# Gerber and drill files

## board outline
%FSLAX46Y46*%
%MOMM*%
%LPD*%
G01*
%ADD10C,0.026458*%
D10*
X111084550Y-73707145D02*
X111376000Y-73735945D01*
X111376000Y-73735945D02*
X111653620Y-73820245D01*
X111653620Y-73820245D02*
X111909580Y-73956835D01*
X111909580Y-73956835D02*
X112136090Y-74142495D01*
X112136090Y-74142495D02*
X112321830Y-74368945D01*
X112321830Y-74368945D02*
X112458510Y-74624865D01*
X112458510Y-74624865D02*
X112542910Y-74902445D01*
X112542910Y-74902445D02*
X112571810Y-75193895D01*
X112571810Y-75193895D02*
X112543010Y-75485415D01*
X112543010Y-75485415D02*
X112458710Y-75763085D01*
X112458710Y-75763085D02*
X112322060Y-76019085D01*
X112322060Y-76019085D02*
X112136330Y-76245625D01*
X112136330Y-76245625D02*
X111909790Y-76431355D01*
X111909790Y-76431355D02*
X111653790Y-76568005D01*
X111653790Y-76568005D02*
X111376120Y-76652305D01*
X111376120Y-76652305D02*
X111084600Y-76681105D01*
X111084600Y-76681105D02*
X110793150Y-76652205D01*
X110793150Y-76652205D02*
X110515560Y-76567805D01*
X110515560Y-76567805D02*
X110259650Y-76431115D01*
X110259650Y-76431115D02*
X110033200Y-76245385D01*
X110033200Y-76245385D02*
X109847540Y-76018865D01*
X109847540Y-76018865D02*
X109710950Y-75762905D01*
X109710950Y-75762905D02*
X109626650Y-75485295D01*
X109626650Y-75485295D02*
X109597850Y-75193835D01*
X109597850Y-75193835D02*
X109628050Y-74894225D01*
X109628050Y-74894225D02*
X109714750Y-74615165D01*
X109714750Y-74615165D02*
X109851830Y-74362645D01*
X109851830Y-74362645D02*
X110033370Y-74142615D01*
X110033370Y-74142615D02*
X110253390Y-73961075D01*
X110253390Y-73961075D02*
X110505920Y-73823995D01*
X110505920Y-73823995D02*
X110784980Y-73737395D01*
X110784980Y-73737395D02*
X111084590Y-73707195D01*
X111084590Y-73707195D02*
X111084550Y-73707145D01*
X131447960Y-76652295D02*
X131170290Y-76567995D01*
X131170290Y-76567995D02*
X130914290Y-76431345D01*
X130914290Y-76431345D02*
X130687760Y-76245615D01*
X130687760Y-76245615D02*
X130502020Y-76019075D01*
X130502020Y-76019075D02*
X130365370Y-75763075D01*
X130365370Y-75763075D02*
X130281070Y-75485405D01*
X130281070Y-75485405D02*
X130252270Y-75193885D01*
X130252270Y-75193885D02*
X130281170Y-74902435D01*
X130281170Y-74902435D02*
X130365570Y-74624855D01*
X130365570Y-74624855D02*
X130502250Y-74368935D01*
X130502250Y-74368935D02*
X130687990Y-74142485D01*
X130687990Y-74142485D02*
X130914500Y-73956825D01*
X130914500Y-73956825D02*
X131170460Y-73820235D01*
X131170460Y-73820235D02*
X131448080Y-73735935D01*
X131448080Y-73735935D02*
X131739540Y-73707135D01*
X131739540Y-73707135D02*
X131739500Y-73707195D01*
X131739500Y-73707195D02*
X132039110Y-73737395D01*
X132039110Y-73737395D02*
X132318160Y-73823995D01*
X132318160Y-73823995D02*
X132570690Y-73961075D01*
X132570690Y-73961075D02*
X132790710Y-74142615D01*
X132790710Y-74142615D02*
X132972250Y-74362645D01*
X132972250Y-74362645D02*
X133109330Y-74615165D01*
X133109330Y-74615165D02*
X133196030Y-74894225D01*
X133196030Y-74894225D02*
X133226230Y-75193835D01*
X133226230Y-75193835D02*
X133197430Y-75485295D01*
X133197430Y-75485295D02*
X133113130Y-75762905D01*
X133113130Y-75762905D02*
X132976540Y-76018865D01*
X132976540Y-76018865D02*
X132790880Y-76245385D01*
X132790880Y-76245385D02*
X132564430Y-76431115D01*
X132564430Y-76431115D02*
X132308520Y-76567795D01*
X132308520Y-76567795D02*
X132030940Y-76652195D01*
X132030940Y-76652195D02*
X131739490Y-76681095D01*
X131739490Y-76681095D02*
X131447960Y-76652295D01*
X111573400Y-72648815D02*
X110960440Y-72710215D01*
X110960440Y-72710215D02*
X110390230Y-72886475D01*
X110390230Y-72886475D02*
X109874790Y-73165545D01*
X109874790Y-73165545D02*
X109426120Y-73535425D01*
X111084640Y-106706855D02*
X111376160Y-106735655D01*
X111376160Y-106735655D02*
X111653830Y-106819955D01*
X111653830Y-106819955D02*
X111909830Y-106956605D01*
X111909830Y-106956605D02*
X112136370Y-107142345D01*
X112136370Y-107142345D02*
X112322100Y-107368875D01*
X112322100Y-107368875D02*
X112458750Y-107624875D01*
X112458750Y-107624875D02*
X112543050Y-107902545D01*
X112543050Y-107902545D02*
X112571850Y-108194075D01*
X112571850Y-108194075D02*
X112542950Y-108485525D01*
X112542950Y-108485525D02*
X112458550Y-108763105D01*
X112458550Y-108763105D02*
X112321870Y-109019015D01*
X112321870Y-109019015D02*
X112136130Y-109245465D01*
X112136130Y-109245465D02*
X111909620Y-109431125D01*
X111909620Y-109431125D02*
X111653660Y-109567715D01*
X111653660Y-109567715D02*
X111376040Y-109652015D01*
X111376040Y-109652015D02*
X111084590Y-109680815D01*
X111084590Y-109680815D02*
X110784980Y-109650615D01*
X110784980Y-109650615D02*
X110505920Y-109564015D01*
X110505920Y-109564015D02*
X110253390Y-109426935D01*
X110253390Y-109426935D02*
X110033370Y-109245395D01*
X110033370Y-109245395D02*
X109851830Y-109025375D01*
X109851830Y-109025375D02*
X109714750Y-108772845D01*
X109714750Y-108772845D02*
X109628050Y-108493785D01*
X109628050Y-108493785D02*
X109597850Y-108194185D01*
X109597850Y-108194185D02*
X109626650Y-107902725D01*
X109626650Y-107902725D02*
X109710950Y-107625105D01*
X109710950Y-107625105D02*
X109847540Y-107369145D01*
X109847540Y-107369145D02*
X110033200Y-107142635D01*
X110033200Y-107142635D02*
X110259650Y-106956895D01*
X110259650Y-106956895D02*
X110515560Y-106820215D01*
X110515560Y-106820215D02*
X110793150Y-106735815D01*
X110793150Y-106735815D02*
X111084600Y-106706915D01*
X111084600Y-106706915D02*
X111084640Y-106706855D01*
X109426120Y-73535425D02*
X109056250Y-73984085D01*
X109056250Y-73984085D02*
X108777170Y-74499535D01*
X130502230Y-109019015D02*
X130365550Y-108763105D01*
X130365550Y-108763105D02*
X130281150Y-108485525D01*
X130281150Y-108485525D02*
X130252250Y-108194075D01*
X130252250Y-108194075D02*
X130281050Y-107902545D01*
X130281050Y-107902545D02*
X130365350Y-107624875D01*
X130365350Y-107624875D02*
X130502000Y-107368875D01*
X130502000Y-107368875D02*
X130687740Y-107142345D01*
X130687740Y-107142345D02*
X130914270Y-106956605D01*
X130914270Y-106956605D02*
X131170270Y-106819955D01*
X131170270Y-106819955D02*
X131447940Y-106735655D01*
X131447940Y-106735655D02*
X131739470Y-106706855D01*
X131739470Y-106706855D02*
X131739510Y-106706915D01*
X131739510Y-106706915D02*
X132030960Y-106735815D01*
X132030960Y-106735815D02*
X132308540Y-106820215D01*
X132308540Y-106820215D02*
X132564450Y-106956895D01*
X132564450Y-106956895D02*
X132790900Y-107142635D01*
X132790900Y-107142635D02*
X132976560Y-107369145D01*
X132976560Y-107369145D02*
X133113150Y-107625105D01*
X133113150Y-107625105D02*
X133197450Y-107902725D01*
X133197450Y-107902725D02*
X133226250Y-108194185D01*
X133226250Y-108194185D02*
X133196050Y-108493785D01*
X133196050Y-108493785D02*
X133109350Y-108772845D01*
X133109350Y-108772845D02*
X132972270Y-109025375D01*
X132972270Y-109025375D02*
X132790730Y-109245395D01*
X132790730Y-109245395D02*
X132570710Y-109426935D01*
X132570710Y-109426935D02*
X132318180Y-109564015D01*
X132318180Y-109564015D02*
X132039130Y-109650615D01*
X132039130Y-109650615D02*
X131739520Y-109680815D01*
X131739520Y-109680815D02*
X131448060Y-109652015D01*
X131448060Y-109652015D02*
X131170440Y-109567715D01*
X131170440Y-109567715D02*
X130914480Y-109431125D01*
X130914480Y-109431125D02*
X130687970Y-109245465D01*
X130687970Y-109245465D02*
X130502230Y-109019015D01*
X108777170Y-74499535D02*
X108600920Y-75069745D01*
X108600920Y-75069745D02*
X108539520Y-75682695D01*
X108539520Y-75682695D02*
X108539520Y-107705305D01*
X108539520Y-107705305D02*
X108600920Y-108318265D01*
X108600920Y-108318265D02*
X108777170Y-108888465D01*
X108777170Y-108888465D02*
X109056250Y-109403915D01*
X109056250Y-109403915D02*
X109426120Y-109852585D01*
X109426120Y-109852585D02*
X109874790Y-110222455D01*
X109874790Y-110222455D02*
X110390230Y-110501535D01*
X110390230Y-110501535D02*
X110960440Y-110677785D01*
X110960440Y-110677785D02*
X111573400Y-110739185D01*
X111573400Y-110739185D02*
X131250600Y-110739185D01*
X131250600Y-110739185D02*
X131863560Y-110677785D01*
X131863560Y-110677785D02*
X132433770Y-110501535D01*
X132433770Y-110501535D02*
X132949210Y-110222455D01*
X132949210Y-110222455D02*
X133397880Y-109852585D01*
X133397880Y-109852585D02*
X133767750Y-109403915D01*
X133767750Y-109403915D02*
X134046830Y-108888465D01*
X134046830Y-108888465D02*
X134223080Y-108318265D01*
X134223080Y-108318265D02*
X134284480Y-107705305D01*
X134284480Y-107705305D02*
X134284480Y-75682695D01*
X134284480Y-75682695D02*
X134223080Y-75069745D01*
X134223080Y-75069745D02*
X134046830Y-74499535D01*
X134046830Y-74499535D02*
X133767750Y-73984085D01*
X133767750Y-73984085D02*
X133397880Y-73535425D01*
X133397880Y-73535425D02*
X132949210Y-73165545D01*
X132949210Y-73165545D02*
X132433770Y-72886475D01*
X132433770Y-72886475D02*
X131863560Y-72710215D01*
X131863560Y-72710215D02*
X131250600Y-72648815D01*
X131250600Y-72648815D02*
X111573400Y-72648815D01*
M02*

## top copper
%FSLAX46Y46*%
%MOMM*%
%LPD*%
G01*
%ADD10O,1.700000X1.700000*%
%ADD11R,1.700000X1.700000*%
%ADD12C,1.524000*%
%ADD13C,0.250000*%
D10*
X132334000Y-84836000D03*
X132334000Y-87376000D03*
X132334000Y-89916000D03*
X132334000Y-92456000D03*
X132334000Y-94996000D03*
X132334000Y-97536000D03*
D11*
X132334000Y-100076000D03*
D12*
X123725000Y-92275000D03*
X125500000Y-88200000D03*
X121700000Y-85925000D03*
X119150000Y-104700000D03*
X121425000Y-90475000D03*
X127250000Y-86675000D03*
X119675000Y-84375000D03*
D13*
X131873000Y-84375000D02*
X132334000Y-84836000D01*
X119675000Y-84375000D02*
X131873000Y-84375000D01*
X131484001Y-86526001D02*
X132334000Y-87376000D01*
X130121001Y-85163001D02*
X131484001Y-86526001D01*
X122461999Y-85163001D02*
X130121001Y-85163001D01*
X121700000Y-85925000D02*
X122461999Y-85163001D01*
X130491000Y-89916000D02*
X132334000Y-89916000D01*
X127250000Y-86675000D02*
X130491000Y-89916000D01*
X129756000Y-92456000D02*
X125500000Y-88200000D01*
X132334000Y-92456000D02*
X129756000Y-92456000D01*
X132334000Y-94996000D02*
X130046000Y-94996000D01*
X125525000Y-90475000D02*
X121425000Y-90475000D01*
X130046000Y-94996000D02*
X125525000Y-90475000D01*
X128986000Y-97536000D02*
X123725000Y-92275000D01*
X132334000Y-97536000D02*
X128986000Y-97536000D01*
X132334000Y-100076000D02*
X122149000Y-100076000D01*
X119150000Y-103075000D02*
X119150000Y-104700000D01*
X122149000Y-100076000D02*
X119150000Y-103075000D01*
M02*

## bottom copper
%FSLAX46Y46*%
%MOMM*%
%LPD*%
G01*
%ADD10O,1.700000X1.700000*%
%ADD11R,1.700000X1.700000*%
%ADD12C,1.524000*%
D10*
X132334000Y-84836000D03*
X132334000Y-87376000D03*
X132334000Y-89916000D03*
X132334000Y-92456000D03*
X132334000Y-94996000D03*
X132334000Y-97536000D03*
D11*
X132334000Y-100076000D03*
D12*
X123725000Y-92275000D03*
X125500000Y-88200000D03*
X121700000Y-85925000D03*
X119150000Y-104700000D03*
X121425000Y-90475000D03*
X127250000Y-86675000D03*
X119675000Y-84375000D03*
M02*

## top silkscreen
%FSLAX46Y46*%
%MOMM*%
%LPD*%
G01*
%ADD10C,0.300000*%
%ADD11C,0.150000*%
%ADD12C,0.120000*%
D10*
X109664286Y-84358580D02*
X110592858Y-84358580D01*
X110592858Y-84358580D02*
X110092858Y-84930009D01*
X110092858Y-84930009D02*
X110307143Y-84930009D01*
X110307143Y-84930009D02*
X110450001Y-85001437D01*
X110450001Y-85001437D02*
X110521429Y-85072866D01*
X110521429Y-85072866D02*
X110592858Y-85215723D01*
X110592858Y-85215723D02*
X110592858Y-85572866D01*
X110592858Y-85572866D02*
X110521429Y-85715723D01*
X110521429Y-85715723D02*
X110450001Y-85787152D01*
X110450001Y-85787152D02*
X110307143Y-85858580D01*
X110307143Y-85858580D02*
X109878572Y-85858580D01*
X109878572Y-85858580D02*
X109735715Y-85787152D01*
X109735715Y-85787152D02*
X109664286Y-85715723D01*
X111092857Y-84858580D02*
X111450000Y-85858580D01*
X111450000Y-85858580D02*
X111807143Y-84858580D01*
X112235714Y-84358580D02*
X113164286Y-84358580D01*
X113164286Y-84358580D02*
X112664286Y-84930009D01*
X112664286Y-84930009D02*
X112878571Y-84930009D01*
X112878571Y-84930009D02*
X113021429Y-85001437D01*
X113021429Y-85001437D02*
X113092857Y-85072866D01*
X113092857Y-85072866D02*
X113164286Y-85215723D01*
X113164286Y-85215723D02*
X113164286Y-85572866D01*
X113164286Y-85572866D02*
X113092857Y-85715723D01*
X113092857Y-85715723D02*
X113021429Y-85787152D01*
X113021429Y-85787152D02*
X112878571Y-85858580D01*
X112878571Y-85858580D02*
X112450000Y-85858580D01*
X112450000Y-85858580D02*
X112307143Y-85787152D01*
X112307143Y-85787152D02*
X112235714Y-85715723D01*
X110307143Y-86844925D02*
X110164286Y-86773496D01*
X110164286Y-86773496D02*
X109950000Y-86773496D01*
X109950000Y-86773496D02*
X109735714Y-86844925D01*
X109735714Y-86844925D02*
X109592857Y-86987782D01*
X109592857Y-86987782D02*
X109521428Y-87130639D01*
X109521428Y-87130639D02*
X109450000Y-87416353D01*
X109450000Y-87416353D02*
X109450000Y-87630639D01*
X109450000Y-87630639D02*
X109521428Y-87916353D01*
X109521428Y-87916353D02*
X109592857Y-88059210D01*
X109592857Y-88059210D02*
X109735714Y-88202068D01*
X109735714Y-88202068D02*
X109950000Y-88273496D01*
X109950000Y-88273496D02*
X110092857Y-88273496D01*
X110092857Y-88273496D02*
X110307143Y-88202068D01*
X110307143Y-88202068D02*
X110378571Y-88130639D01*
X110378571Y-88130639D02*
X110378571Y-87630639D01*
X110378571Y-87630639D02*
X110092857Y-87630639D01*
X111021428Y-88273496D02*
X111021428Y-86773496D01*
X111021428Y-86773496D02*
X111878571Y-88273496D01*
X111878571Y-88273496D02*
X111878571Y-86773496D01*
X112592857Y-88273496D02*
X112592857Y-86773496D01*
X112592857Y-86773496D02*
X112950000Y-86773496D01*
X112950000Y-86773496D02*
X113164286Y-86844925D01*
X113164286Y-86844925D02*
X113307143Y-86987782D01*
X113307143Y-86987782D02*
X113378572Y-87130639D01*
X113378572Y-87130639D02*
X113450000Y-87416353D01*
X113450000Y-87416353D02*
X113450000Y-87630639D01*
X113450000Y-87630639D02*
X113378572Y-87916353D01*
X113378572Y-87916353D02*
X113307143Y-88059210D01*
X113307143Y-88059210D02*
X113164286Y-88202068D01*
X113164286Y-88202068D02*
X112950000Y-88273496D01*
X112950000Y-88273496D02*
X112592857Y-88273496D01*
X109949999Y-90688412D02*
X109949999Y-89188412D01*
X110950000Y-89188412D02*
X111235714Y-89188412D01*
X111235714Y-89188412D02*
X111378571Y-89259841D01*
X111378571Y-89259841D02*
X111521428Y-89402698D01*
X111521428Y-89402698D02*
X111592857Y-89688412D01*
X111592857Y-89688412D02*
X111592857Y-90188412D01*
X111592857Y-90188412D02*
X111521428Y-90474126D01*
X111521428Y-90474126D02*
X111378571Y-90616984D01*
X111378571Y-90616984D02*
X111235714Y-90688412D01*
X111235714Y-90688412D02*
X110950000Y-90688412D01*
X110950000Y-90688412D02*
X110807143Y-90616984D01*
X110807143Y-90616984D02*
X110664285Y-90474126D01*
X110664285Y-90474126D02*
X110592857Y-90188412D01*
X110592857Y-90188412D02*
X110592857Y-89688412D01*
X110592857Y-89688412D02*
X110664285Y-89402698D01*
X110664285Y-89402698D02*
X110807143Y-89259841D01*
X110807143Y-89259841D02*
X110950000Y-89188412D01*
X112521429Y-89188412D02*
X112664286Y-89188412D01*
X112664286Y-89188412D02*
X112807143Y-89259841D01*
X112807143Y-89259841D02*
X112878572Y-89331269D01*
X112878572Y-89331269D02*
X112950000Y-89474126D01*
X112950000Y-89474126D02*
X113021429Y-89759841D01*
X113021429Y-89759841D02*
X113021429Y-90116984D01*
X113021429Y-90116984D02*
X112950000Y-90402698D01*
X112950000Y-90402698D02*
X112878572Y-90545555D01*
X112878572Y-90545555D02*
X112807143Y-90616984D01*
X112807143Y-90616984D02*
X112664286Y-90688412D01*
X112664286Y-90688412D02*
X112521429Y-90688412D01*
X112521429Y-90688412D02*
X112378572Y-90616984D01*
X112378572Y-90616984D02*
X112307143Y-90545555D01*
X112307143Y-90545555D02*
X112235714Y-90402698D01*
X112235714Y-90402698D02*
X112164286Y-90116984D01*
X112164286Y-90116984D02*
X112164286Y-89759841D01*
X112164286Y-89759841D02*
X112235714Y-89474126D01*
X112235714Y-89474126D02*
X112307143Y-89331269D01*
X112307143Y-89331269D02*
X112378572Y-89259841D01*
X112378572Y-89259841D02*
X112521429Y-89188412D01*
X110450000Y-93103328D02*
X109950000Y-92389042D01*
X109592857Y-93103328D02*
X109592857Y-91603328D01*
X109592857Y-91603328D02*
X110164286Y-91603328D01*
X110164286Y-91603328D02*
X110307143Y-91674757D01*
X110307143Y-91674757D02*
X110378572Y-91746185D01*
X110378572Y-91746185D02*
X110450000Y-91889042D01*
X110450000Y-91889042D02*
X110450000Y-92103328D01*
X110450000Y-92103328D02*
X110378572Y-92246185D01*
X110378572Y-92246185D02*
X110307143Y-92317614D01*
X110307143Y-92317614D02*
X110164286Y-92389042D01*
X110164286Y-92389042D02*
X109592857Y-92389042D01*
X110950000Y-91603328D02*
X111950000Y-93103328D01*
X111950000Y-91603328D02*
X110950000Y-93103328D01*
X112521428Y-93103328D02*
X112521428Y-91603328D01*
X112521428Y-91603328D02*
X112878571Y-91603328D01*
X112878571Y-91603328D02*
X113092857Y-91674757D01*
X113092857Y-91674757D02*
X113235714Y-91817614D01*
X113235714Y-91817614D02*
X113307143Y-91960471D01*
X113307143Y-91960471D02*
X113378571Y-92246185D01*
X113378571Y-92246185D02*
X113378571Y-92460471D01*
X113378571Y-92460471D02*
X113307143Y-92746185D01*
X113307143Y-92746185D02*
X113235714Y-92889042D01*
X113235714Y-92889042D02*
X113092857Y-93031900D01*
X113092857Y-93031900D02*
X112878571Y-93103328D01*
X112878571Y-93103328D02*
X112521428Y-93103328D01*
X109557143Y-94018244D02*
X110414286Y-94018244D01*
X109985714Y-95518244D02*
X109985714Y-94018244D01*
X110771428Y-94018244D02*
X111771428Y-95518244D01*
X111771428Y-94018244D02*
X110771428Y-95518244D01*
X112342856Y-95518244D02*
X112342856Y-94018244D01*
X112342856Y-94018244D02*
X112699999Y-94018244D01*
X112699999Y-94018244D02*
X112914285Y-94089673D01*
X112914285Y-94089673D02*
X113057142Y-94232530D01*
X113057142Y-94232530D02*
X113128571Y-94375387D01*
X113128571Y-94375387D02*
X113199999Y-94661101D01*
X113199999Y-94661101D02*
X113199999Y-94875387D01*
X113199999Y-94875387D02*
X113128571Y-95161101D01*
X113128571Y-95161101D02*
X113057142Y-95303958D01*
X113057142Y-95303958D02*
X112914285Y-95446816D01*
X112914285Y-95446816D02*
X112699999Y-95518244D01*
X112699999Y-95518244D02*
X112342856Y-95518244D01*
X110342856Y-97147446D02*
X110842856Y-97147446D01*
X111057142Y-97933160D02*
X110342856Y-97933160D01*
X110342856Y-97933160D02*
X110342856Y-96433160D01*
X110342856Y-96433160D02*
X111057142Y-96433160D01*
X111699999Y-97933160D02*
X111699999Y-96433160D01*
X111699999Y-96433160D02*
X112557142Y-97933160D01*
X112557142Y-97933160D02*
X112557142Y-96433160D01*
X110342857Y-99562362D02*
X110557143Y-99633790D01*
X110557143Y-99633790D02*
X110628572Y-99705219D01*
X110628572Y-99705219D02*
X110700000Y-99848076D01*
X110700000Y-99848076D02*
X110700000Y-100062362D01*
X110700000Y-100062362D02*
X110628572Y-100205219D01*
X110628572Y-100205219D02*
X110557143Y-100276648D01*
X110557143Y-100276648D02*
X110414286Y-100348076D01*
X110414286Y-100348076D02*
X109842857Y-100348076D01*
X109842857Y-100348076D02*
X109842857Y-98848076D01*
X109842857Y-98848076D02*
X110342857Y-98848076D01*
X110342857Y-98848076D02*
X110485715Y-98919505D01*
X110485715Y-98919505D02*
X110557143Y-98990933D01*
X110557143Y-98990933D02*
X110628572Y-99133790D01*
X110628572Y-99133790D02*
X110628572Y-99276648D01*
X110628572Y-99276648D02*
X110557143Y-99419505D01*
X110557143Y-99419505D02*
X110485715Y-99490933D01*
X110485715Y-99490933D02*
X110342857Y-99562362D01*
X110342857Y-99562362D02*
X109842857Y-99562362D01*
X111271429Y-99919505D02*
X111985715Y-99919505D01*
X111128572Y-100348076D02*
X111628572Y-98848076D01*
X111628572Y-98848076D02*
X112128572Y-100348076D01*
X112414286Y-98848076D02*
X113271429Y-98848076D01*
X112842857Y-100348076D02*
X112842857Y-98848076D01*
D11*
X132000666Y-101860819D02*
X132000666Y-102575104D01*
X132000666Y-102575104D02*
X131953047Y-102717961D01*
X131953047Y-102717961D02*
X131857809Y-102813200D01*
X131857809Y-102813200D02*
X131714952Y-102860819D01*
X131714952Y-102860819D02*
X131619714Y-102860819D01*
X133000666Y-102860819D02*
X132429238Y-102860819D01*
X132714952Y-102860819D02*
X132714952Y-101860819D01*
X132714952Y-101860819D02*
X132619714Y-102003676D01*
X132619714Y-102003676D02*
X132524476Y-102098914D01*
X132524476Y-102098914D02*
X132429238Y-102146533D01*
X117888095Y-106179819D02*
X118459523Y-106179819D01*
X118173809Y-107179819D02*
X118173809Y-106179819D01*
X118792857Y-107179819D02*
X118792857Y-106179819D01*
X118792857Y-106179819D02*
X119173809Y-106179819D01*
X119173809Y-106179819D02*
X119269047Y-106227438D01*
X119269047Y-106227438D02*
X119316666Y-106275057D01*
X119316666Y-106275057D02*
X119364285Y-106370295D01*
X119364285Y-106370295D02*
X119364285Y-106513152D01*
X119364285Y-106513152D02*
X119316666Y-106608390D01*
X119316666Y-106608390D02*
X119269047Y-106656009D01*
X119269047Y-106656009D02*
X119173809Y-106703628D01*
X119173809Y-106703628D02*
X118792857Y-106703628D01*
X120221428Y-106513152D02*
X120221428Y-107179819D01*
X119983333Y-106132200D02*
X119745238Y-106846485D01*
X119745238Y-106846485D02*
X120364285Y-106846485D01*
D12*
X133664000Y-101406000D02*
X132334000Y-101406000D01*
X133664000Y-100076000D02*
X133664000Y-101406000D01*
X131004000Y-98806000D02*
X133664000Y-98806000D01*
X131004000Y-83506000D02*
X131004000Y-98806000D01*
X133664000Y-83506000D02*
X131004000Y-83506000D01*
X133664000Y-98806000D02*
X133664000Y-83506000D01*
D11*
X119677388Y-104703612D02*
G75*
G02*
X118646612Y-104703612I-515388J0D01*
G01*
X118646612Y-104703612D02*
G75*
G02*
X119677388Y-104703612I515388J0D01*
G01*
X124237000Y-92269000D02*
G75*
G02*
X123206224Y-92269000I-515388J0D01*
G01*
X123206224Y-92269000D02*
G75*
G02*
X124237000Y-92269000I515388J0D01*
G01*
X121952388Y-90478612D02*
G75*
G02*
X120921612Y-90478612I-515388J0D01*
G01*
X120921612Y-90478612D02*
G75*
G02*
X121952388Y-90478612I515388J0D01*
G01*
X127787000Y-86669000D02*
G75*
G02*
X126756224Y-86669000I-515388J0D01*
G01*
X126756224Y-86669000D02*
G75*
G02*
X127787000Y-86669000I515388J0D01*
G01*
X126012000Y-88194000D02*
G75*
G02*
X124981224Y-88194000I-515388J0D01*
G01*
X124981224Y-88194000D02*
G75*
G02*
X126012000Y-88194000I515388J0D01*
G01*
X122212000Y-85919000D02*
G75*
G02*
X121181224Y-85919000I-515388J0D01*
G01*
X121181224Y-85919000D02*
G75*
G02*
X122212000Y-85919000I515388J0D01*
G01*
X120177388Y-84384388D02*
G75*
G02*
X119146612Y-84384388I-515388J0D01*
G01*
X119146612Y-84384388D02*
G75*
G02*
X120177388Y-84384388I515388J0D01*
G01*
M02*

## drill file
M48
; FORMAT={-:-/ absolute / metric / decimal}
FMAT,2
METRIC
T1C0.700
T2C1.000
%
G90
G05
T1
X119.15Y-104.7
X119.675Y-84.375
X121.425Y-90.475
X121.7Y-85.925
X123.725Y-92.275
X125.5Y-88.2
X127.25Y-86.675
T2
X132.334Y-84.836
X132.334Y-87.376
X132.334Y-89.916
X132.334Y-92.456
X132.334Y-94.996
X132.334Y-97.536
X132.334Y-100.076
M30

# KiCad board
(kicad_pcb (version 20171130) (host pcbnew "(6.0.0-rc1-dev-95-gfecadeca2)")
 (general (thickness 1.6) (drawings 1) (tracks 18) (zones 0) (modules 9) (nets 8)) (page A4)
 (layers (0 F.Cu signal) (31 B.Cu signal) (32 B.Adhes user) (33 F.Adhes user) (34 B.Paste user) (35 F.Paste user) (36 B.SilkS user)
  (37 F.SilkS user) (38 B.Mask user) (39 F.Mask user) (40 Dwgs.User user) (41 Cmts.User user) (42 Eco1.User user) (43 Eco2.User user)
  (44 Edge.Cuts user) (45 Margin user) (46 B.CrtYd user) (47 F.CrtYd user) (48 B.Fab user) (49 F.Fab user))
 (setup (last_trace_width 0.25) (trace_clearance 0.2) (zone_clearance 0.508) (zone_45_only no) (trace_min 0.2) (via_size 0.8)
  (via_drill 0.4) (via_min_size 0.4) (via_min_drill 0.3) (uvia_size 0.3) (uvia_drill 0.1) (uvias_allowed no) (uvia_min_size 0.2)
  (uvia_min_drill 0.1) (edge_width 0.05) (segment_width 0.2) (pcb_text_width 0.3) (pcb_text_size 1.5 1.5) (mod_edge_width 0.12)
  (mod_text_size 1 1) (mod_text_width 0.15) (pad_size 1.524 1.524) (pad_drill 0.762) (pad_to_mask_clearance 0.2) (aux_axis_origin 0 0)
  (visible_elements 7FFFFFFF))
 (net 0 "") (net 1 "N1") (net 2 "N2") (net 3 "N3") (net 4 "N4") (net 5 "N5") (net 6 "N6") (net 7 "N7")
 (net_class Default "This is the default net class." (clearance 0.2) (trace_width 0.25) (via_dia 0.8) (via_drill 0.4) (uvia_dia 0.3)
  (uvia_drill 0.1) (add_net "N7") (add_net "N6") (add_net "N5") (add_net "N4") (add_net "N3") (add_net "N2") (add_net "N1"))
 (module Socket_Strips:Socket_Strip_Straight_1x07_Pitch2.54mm (layer F.Cu) (at 132.334 100.076 180)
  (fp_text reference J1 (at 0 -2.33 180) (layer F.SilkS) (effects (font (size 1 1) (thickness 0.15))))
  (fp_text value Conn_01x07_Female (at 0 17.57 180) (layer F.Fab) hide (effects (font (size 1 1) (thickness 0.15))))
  (fp_line (start -1.33 -1.33) (end 0 -1.33) (layer F.SilkS) (width 0.12))
  (fp_line (start -1.33 0) (end -1.33 -1.33) (layer F.SilkS) (width 0.12))
  (fp_line (start 1.33 1.27) (end -1.33 1.27) (layer F.SilkS) (width 0.12))
  (fp_line (start 1.33 16.57) (end 1.33 1.27) (layer F.SilkS) (width 0.12))
  (fp_line (start -1.33 16.57) (end 1.33 16.57) (layer F.SilkS) (width 0.12))
  (fp_line (start -1.33 1.27) (end -1.33 16.57) (layer F.SilkS) (width 0.12))
  (pad 7 thru_hole oval (at 0 15.24 180) (size 1.7 1.7) (drill 1) (layers *.Cu *.Mask) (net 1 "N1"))
  (pad 6 thru_hole oval (at 0 12.7 180) (size 1.7 1.7) (drill 1) (layers *.Cu *.Mask) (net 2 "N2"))
  (pad 5 thru_hole oval (at 0 10.16 180) (size 1.7 1.7) (drill 1) (layers *.Cu *.Mask) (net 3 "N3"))
  (pad 4 thru_hole oval (at 0 7.62 180) (size 1.7 1.7) (drill 1) (layers *.Cu *.Mask) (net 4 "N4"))
  (pad 3 thru_hole oval (at 0 5.08 180) (size 1.7 1.7) (drill 1) (layers *.Cu *.Mask) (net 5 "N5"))
  (pad 2 thru_hole oval (at 0 2.54 180) (size 1.7 1.7) (drill 1) (layers *.Cu *.Mask) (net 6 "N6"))
  (pad 1 thru_hole rect (at 0 0 180) (size 1.7 1.7) (drill 1) (layers *.Cu *.Mask) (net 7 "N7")))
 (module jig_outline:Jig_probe (layer F.Cu) (at 121.412 91.694)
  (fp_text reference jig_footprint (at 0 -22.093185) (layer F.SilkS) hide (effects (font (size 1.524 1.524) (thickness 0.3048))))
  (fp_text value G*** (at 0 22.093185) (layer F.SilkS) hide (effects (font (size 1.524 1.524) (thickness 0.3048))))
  (fp_circle (center -2.25 13.009612) (end -1.925 12.609612) (layer F.SilkS) (width 0.15))
  (fp_circle (center 2.309612 0.575) (end 2.634612 0.175) (layer F.SilkS) (width 0.15))
  (fp_circle (center 0.025 -1.215388) (end 0.540388 -1.215388) (layer F.SilkS) (width 0.15))
  (fp_circle (center 5.859612 -5.025) (end 6.184612 -5.425) (layer F.SilkS) (width 0.15))
  (fp_circle (center 4.084612 -3.5) (end 4.409612 -3.9) (layer F.SilkS) (width 0.15))
  (fp_circle (center 0.284612 -5.775) (end 0.609612 -6.175) (layer F.SilkS) (width 0.15))
  (fp_circle (center -1.75 -7.309612) (end -1.425 -7.709612) (layer F.SilkS) (width 0.15))
  (fp_line (start -10.32745 -17.986855) (end -10.036 -17.958055) (layer Edge.Cuts) (width 0.026458))
  (fp_line (start -10.036 -17.958055) (end -9.75838 -17.873755) (layer Edge.Cuts) (width 0.026458))
  (fp_line (start -9.75838 -17.873755) (end -9.50242 -17.737165) (layer Edge.Cuts) (width 0.026458))
  (fp_line (start -9.50242 -17.737165) (end -9.27591 -17.551505) (layer Edge.Cuts) (width 0.026458))
  (fp_line (start -9.27591 -17.551505) (end -9.09017 -17.325055) (layer Edge.Cuts) (width 0.026458))
  (fp_line (start -9.09017 -17.325055) (end -8.95349 -17.069135) (layer Edge.Cuts) (width 0.026458))
  (fp_line (start -8.95349 -17.069135) (end -8.86909 -16.791555) (layer Edge.Cuts) (width 0.026458))
  (fp_line (start -8.86909 -16.791555) (end -8.84019 -16.500105) (layer Edge.Cuts) (width 0.026458))
  (fp_line (start -8.84019 -16.500105) (end -8.86899 -16.208585) (layer Edge.Cuts) (width 0.026458))
  (fp_line (start -8.86899 -16.208585) (end -8.95329 -15.930915) (layer Edge.Cuts) (width 0.026458))
  (fp_line (start -8.95329 -15.930915) (end -9.08994 -15.674915) (layer Edge.Cuts) (width 0.026458))
  (fp_line (start -9.08994 -15.674915) (end -9.27567 -15.448375) (layer Edge.Cuts) (width 0.026458))
  (fp_line (start -9.27567 -15.448375) (end -9.50221 -15.262645) (layer Edge.Cuts) (width 0.026458))
  (fp_line (start -9.50221 -15.262645) (end -9.75821 -15.125995) (layer Edge.Cuts) (width 0.026458))
  (fp_line (start -9.75821 -15.125995) (end -10.03588 -15.041695) (layer Edge.Cuts) (width 0.026458))
  (fp_line (start -10.03588 -15.041695) (end -10.3274 -15.012895) (layer Edge.Cuts) (width 0.026458))
  (fp_line (start -10.3274 -15.012895) (end -10.61885 -15.041795) (layer Edge.Cuts) (width 0.026458))
  (fp_line (start -10.61885 -15.041795) (end -10.89644 -15.126195) (layer Edge.Cuts) (width 0.026458))
  (fp_line (start -10.89644 -15.126195) (end -11.15235 -15.262885) (layer Edge.Cuts) (width 0.026458))
  (fp_line (start -11.15235 -15.262885) (end -11.3788 -15.448615) (layer Edge.Cuts) (width 0.026458))
  (fp_line (start -11.3788 -15.448615) (end -11.56446 -15.675135) (layer Edge.Cuts) (width 0.026458))
  (fp_line (start -11.56446 -15.675135) (end -11.70105 -15.931095) (layer Edge.Cuts) (width 0.026458))
  (fp_line (start -11.70105 -15.931095) (end -11.78535 -16.208705) (layer Edge.Cuts) (width 0.026458))
  (fp_line (start -11.78535 -16.208705) (end -11.81415 -16.500165) (layer Edge.Cuts) (width 0.026458))
  (fp_line (start -11.81415 -16.500165) (end -11.78395 -16.799775) (layer Edge.Cuts) (width 0.026458))
  (fp_line (start -11.78395 -16.799775) (end -11.69725 -17.078835) (layer Edge.Cuts) (width 0.026458))
  (fp_line (start -11.69725 -17.078835) (end -11.56017 -17.331355) (layer Edge.Cuts) (width 0.026458))
  (fp_line (start -11.56017 -17.331355) (end -11.37863 -17.551385) (layer Edge.Cuts) (width 0.026458))
  (fp_line (start -11.37863 -17.551385) (end -11.15861 -17.732925) (layer Edge.Cuts) (width 0.026458))
  (fp_line (start -11.15861 -17.732925) (end -10.90608 -17.870005) (layer Edge.Cuts) (width 0.026458))
  (fp_line (start -10.90608 -17.870005) (end -10.62702 -17.956605) (layer Edge.Cuts) (width 0.026458))
  (fp_line (start -10.62702 -17.956605) (end -10.32741 -17.986805) (layer Edge.Cuts) (width 0.026458))
  (fp_line (start -10.32741 -17.986805) (end -10.32745 -17.986855) (layer Edge.Cuts) (width 0.026458))
  (fp_line (start 10.03596 -15.041705) (end 9.75829 -15.126005) (layer Edge.Cuts) (width 0.026458))
  (fp_line (start 9.75829 -15.126005) (end 9.50229 -15.262655) (layer Edge.Cuts) (width 0.026458))
  (fp_line (start 9.50229 -15.262655) (end 9.27576 -15.448385) (layer Edge.Cuts) (width 0.026458))
  (fp_line (start 9.27576 -15.448385) (end 9.09002 -15.674925) (layer Edge.Cuts) (width 0.026458))
  (fp_line (start 9.09002 -15.674925) (end 8.95337 -15.930925) (layer Edge.Cuts) (width 0.026458))
  (fp_line (start 8.95337 -15.930925) (end 8.86907 -16.208595) (layer Edge.Cuts) (width 0.026458))
  (fp_line (start 8.86907 -16.208595) (end 8.84027 -16.500115) (layer Edge.Cuts) (width 0.026458))
  (fp_line (start 8.84027 -16.500115) (end 8.86917 -16.791565) (layer Edge.Cuts) (width 0.026458))
  (fp_line (start 8.86917 -16.791565) (end 8.95357 -17.069145) (layer Edge.Cuts) (width 0.026458))
  (fp_line (start 8.95357 -17.069145) (end 9.09025 -17.325065) (layer Edge.Cuts) (width 0.026458))
  (fp_line (start 9.09025 -17.325065) (end 9.27599 -17.551515) (layer Edge.Cuts) (width 0.026458))
  (fp_line (start 9.27599 -17.551515) (end 9.5025 -17.737175) (layer Edge.Cuts) (width 0.026458))
  (fp_line (start 9.5025 -17.737175) (end 9.75846 -17.873765) (layer Edge.Cuts) (width 0.026458))
  (fp_line (start 9.75846 -17.873765) (end 10.03608 -17.958065) (layer Edge.Cuts) (width 0.026458))
  (fp_line (start 10.03608 -17.958065) (end 10.32754 -17.986865) (layer Edge.Cuts) (width 0.026458))
  (fp_line (start 10.32754 -17.986865) (end 10.3275 -17.986805) (layer Edge.Cuts) (width 0.026458))
  (fp_line (start 10.3275 -17.986805) (end 10.62711 -17.956605) (layer Edge.Cuts) (width 0.026458))
  (fp_line (start 10.62711 -17.956605) (end 10.90616 -17.870005) (layer Edge.Cuts) (width 0.026458))
  (fp_line (start 10.90616 -17.870005) (end 11.15869 -17.732925) (layer Edge.Cuts) (width 0.026458))
  (fp_line (start 11.15869 -17.732925) (end 11.37871 -17.551385) (layer Edge.Cuts) (width 0.026458))
  (fp_line (start 11.37871 -17.551385) (end 11.56025 -17.331355) (layer Edge.Cuts) (width 0.026458))
  (fp_line (start 11.56025 -17.331355) (end 11.69733 -17.078835) (layer Edge.Cuts) (width 0.026458))
  (fp_line (start 11.69733 -17.078835) (end 11.78403 -16.799775) (layer Edge.Cuts) (width 0.026458))
  (fp_line (start 11.78403 -16.799775) (end 11.81423 -16.500165) (layer Edge.Cuts) (width 0.026458))
  (fp_line (start 11.81423 -16.500165) (end 11.78543 -16.208705) (layer Edge.Cuts) (width 0.026458))
  (fp_line (start 11.78543 -16.208705) (end 11.70113 -15.931095) (layer Edge.Cuts) (width 0.026458))
  (fp_line (start 11.70113 -15.931095) (end 11.56454 -15.675135) (layer Edge.Cuts) (width 0.026458))
  (fp_line (start 11.56454 -15.675135) (end 11.37888 -15.448615) (layer Edge.Cuts) (width 0.026458))
  (fp_line (start 11.37888 -15.448615) (end 11.15243 -15.262885) (layer Edge.Cuts) (width 0.026458))
  (fp_line (start 11.15243 -15.262885) (end 10.89652 -15.126205) (layer Edge.Cuts) (width 0.026458))
  (fp_line (start 10.89652 -15.126205) (end 10.61894 -15.041805) (layer Edge.Cuts) (width 0.026458))
  (fp_line (start 10.61894 -15.041805) (end 10.32749 -15.012905) (layer Edge.Cuts) (width 0.026458))
  (fp_line (start 10.32749 -15.012905) (end 10.03596 -15.041705) (layer Edge.Cuts) (width 0.026458))
  (fp_line (start -9.8386 -19.045185) (end -10.45156 -18.983785) (layer Edge.Cuts) (width 0.026458))
  (fp_line (start -10.45156 -18.983785) (end -11.02177 -18.807525) (layer Edge.Cuts) (width 0.026458))
  (fp_line (start -11.02177 -18.807525) (end -11.53721 -18.528455) (layer Edge.Cuts) (width 0.026458))
  (fp_line (start -11.53721 -18.528455) (end -11.98588 -18.158575) (layer Edge.Cuts) (width 0.026458))
  (fp_line (start -10.32736 15.012855) (end -10.03584 15.041655) (layer Edge.Cuts) (width 0.026458))
  (fp_line (start -10.03584 15.041655) (end -9.75817 15.125955) (layer Edge.Cuts) (width 0.026458))
  (fp_line (start -9.75817 15.125955) (end -9.50217 15.262605) (layer Edge.Cuts) (width 0.026458))
  (fp_line (start -9.50217 15.262605) (end -9.27563 15.448345) (layer Edge.Cuts) (width 0.026458))
  (fp_line (start -9.27563 15.448345) (end -9.0899 15.674875) (layer Edge.Cuts) (width 0.026458))
  (fp_line (start -9.0899 15.674875) (end -8.95325 15.930875) (layer Edge.Cuts) (width 0.026458))
  (fp_line (start -8.95325 15.930875) (end -8.86895 16.208545) (layer Edge.Cuts) (width 0.026458))
  (fp_line (start -8.86895 16.208545) (end -8.84015 16.500075) (layer Edge.Cuts) (width 0.026458))
  (fp_line (start -8.84015 16.500075) (end -8.86905 16.791525) (layer Edge.Cuts) (width 0.026458))
  (fp_line (start -8.86905 16.791525) (end -8.95345 17.069105) (layer Edge.Cuts) (width 0.026458))
  (fp_line (start -8.95345 17.069105) (end -9.09013 17.325015) (layer Edge.Cuts) (width 0.026458))
  (fp_line (start -9.09013 17.325015) (end -9.27587 17.551465) (layer Edge.Cuts) (width 0.026458))
  (fp_line (start -9.27587 17.551465) (end -9.50238 17.737125) (layer Edge.Cuts) (width 0.026458))
  (fp_line (start -9.50238 17.737125) (end -9.75834 17.873715) (layer Edge.Cuts) (width 0.026458))
  (fp_line (start -9.75834 17.873715) (end -10.03596 17.958015) (layer Edge.Cuts) (width 0.026458))
  (fp_line (start -10.03596 17.958015) (end -10.32741 17.986815) (layer Edge.Cuts) (width 0.026458))
  (fp_line (start -10.32741 17.986815) (end -10.62702 17.956615) (layer Edge.Cuts) (width 0.026458))
  (fp_line (start -10.62702 17.956615) (end -10.90608 17.870015) (layer Edge.Cuts) (width 0.026458))
  (fp_line (start -10.90608 17.870015) (end -11.15861 17.732935) (layer Edge.Cuts) (width 0.026458))
  (fp_line (start -11.15861 17.732935) (end -11.37863 17.551395) (layer Edge.Cuts) (width 0.026458))
  (fp_line (start -11.37863 17.551395) (end -11.56017 17.331375) (layer Edge.Cuts) (width 0.026458))
  (fp_line (start -11.56017 17.331375) (end -11.69725 17.078845) (layer Edge.Cuts) (width 0.026458))
  (fp_line (start -11.69725 17.078845) (end -11.78395 16.799785) (layer Edge.Cuts) (width 0.026458))
  (fp_line (start -11.78395 16.799785) (end -11.81415 16.500185) (layer Edge.Cuts) (width 0.026458))
  (fp_line (start -11.81415 16.500185) (end -11.78535 16.208725) (layer Edge.Cuts) (width 0.026458))
  (fp_line (start -11.78535 16.208725) (end -11.70105 15.931105) (layer Edge.Cuts) (width 0.026458))
  (fp_line (start -11.70105 15.931105) (end -11.56446 15.675145) (layer Edge.Cuts) (width 0.026458))
  (fp_line (start -11.56446 15.675145) (end -11.3788 15.448635) (layer Edge.Cuts) (width 0.026458))
  (fp_line (start -11.3788 15.448635) (end -11.15235 15.262895) (layer Edge.Cuts) (width 0.026458))
  (fp_line (start -11.15235 15.262895) (end -10.89644 15.126215) (layer Edge.Cuts) (width 0.026458))
  (fp_line (start -10.89644 15.126215) (end -10.61885 15.041815) (layer Edge.Cuts) (width 0.026458))
  (fp_line (start -10.61885 15.041815) (end -10.3274 15.012915) (layer Edge.Cuts) (width 0.026458))
  (fp_line (start -10.3274 15.012915) (end -10.32736 15.012855) (layer Edge.Cuts) (width 0.026458))
  (fp_line (start -11.98588 -18.158575) (end -12.35575 -17.709915) (layer Edge.Cuts) (width 0.026458))
  (fp_line (start -12.35575 -17.709915) (end -12.63483 -17.194465) (layer Edge.Cuts) (width 0.026458))
  (fp_line (start 9.09023 17.325015) (end 8.95355 17.069105) (layer Edge.Cuts) (width 0.026458))
  (fp_line (start 8.95355 17.069105) (end 8.86915 16.791525) (layer Edge.Cuts) (width 0.026458))
  (fp_line (start 8.86915 16.791525) (end 8.84025 16.500075) (layer Edge.Cuts) (width 0.026458))
  (fp_line (start 8.84025 16.500075) (end 8.86905 16.208545) (layer Edge.Cuts) (width 0.026458))
  (fp_line (start 8.86905 16.208545) (end 8.95335 15.930875) (layer Edge.Cuts) (width 0.026458))
  (fp_line (start 8.95335 15.930875) (end 9.09 15.674875) (layer Edge.Cuts) (width 0.026458))
  (fp_line (start 9.09 15.674875) (end 9.27574 15.448345) (layer Edge.Cuts) (width 0.026458))
  (fp_line (start 9.27574 15.448345) (end 9.50227 15.262605) (layer Edge.Cuts) (width 0.026458))
  (fp_line (start 9.50227 15.262605) (end 9.75827 15.125955) (layer Edge.Cuts) (width 0.026458))
  (fp_line (start 9.75827 15.125955) (end 10.03594 15.041655) (layer Edge.Cuts) (width 0.026458))
  (fp_line (start 10.03594 15.041655) (end 10.32747 15.012855) (layer Edge.Cuts) (width 0.026458))
  (fp_line (start 10.32747 15.012855) (end 10.32751 15.012915) (layer Edge.Cuts) (width 0.026458))
  (fp_line (start 10.32751 15.012915) (end 10.61896 15.041815) (layer Edge.Cuts) (width 0.026458))
  (fp_line (start 10.61896 15.041815) (end 10.89654 15.126215) (layer Edge.Cuts) (width 0.026458))
  (fp_line (start 10.89654 15.126215) (end 11.15245 15.262895) (layer Edge.Cuts) (width 0.026458))
  (fp_line (start 11.15245 15.262895) (end 11.3789 15.448635) (layer Edge.Cuts) (width 0.026458))
  (fp_line (start 11.3789 15.448635) (end 11.56456 15.675145) (layer Edge.Cuts) (width 0.026458))
  (fp_line (start 11.56456 15.675145) (end 11.70115 15.931105) (layer Edge.Cuts) (width 0.026458))
  (fp_line (start 11.70115 15.931105) (end 11.78545 16.208725) (layer Edge.Cuts) (width 0.026458))
  (fp_line (start 11.78545 16.208725) (end 11.81425 16.500185) (layer Edge.Cuts) (width 0.026458))
  (fp_line (start 11.81425 16.500185) (end 11.78405 16.799785) (layer Edge.Cuts) (width 0.026458))
  (fp_line (start 11.78405 16.799785) (end 11.69735 17.078845) (layer Edge.Cuts) (width 0.026458))
  (fp_line (start 11.69735 17.078845) (end 11.56027 17.331375) (layer Edge.Cuts) (width 0.026458))
  (fp_line (start 11.56027 17.331375) (end 11.37873 17.551395) (layer Edge.Cuts) (width 0.026458))
  (fp_line (start 11.37873 17.551395) (end 11.15871 17.732935) (layer Edge.Cuts) (width 0.026458))
  (fp_line (start 11.15871 17.732935) (end 10.90618 17.870015) (layer Edge.Cuts) (width 0.026458))
  (fp_line (start 10.90618 17.870015) (end 10.62713 17.956615) (layer Edge.Cuts) (width 0.026458))
  (fp_line (start 10.62713 17.956615) (end 10.32752 17.986815) (layer Edge.Cuts) (width 0.026458))
  (fp_line (start 10.32752 17.986815) (end 10.03606 17.958015) (layer Edge.Cuts) (width 0.026458))
  (fp_line (start 10.03606 17.958015) (end 9.75844 17.873715) (layer Edge.Cuts) (width 0.026458))
  (fp_line (start 9.75844 17.873715) (end 9.50248 17.737125) (layer Edge.Cuts) (width 0.026458))
  (fp_line (start 9.50248 17.737125) (end 9.27597 17.551465) (layer Edge.Cuts) (width 0.026458))
  (fp_line (start 9.27597 17.551465) (end 9.09023 17.325015) (layer Edge.Cuts) (width 0.026458))
  (fp_line (start -12.63483 -17.194465) (end -12.81108 -16.624255) (layer Edge.Cuts) (width 0.026458))
  (fp_line (start -12.81108 -16.624255) (end -12.87248 -16.011305) (layer Edge.Cuts) (width 0.026458))
  (fp_line (start -12.87248 -16.011305) (end -12.87248 16.011305) (layer Edge.Cuts) (width 0.026458))
  (fp_line (start -12.87248 16.011305) (end -12.81108 16.624265) (layer Edge.Cuts) (width 0.026458))
  (fp_line (start -12.81108 16.624265) (end -12.63483 17.194465) (layer Edge.Cuts) (width 0.026458))
  (fp_line (start -12.63483 17.194465) (end -12.35575 17.709915) (layer Edge.Cuts) (width 0.026458))
  (fp_line (start -12.35575 17.709915) (end -11.98588 18.158585) (layer Edge.Cuts) (width 0.026458))
  (fp_line (start -11.98588 18.158585) (end -11.53721 18.528455) (layer Edge.Cuts) (width 0.026458))
  (fp_line (start -11.53721 18.528455) (end -11.02177 18.807535) (layer Edge.Cuts) (width 0.026458))
  (fp_line (start -11.02177 18.807535) (end -10.45156 18.983785) (layer Edge.Cuts) (width 0.026458))
  (fp_line (start -10.45156 18.983785) (end -9.8386 19.045185) (layer Edge.Cuts) (width 0.026458))
  (fp_line (start -9.8386 19.045185) (end 9.8386 19.045185) (layer Edge.Cuts) (width 0.026458))
  (fp_line (start 9.8386 19.045185) (end 10.45156 18.983785) (layer Edge.Cuts) (width 0.026458))
  (fp_line (start 10.45156 18.983785) (end 11.02177 18.807535) (layer Edge.Cuts) (width 0.026458))
  (fp_line (start 11.02177 18.807535) (end 11.53721 18.528455) (layer Edge.Cuts) (width 0.026458))
  (fp_line (start 11.53721 18.528455) (end 11.98588 18.158585) (layer Edge.Cuts) (width 0.026458))
  (fp_line (start 11.98588 18.158585) (end 12.35575 17.709915) (layer Edge.Cuts) (width 0.026458))
  (fp_line (start 12.35575 17.709915) (end 12.63483 17.194465) (layer Edge.Cuts) (width 0.026458))
  (fp_line (start 12.63483 17.194465) (end 12.81108 16.624265) (layer Edge.Cuts) (width 0.026458))
  (fp_line (start 12.81108 16.624265) (end 12.87248 16.011305) (layer Edge.Cuts) (width 0.026458))
  (fp_line (start 12.87248 16.011305) (end 12.87248 -16.011305) (layer Edge.Cuts) (width 0.026458))
  (fp_line (start 12.87248 -16.011305) (end 12.81108 -16.624255) (layer Edge.Cuts) (width 0.026458))
  (fp_line (start 12.81108 -16.624255) (end 12.63483 -17.194465) (layer Edge.Cuts) (width 0.026458))
  (fp_line (start 12.63483 -17.194465) (end 12.35575 -17.709915) (layer Edge.Cuts) (width 0.026458))
  (fp_line (start 12.35575 -17.709915) (end 11.98588 -18.158575) (layer Edge.Cuts) (width 0.026458))
  (fp_line (start 11.98588 -18.158575) (end 11.53721 -18.528455) (layer Edge.Cuts) (width 0.026458))
  (fp_line (start 11.53721 -18.528455) (end 11.02177 -18.807525) (layer Edge.Cuts) (width 0.026458))
  (fp_line (start 11.02177 -18.807525) (end 10.45156 -18.983785) (layer Edge.Cuts) (width 0.026458))
  (fp_line (start 10.45156 -18.983785) (end 9.8386 -19.045185) (layer Edge.Cuts) (width 0.026458))
  (fp_line (start 9.8386 -19.045185) (end -9.8386 -19.045185) (layer Edge.Cuts) (width 0.026458)))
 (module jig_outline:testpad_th (layer F.Cu) (at 123.725 92.275)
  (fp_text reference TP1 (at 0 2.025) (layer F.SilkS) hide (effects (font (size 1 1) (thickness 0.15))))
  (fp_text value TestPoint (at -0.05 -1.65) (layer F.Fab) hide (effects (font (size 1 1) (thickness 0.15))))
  (pad 1 thru_hole circle (at 0 0) (size 1.524 1.524) (drill 0.7) (layers *.Cu *.Mask) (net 6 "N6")))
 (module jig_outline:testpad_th (layer F.Cu) (at 125.5 88.2)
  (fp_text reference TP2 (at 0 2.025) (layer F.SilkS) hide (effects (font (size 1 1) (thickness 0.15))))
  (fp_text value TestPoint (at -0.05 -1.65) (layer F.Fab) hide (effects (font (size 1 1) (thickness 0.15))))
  (pad 1 thru_hole circle (at 0 0) (size 1.524 1.524) (drill 0.7) (layers *.Cu *.Mask) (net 4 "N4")))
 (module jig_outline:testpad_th (layer F.Cu) (at 121.7 85.925)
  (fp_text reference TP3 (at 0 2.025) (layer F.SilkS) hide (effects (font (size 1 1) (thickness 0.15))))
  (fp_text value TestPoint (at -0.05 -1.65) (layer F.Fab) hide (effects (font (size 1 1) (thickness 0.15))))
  (pad 1 thru_hole circle (at 0 0) (size 1.524 1.524) (drill 0.7) (layers *.Cu *.Mask) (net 2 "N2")))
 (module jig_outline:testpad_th (layer F.Cu) (at 119.15 104.7)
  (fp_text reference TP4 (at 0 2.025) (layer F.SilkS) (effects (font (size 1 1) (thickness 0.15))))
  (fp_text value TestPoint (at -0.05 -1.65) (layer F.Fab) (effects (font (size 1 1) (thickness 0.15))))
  (pad 1 thru_hole circle (at 0 0) (size 1.524 1.524) (drill 0.7) (layers *.Cu *.Mask) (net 7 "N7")))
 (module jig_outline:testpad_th (layer F.Cu) (at 121.425 90.475)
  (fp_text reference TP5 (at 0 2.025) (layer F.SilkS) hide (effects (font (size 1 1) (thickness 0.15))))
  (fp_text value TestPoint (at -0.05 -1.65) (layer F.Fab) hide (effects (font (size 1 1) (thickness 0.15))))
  (pad 1 thru_hole circle (at 0 0) (size 1.524 1.524) (drill 0.7) (layers *.Cu *.Mask) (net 5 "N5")))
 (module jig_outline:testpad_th (layer F.Cu) (at 127.25 86.675)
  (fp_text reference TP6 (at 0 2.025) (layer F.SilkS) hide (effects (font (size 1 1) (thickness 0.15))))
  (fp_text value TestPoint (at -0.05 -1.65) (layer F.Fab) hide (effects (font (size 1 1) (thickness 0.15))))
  (pad 1 thru_hole circle (at 0 0) (size 1.524 1.524) (drill 0.7) (layers *.Cu *.Mask) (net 3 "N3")))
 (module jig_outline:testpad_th (layer F.Cu) (at 119.675 84.375)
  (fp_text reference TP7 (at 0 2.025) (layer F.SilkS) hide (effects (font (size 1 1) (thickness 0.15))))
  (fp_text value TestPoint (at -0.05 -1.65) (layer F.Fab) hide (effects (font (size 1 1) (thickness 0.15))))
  (pad 1 thru_hole circle (at 0 0) (size 1.524 1.524) (drill 0.7) (layers *.Cu *.Mask) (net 1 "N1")))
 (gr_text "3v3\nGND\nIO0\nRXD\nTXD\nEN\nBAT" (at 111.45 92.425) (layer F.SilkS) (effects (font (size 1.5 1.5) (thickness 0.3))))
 (segment (start 131.873 84.375) (end 132.334 84.836) (width 0.25) (layer F.Cu) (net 1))
 (segment (start 119.675 84.375) (end 131.873 84.375) (width 0.25) (layer F.Cu) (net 1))
 (segment (start 131.484001 86.526001) (end 132.334 87.376) (width 0.25) (layer F.Cu) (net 2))
 (segment (start 130.121001 85.163001) (end 131.484001 86.526001) (width 0.25) (layer F.Cu) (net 2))
 (segment (start 122.461999 85.163001) (end 130.121001 85.163001) (width 0.25) (layer F.Cu) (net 2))
 (segment (start 121.7 85.925) (end 122.461999 85.163001) (width 0.25) (layer F.Cu) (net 2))
 (segment (start 130.491 89.916) (end 132.334 89.916) (width 0.25) (layer F.Cu) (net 3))
 (segment (start 127.25 86.675) (end 130.491 89.916) (width 0.25) (layer F.Cu) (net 3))
 (segment (start 129.756 92.456) (end 125.5 88.2) (width 0.25) (layer F.Cu) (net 4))
 (segment (start 132.334 92.456) (end 129.756 92.456) (width 0.25) (layer F.Cu) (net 4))
 (segment (start 132.334 94.996) (end 130.046 94.996) (width 0.25) (layer F.Cu) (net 5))
 (segment (start 125.525 90.475) (end 121.425 90.475) (width 0.25) (layer F.Cu) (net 5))
 (segment (start 130.046 94.996) (end 125.525 90.475) (width 0.25) (layer F.Cu) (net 5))
 (segment (start 128.986 97.536) (end 123.725 92.275) (width 0.25) (layer F.Cu) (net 6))
 (segment (start 132.334 97.536) (end 128.986 97.536) (width 0.25) (layer F.Cu) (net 6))
 (segment (start 132.334 100.076) (end 122.149 100.076) (width 0.25) (layer F.Cu) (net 7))
 (segment (start 119.15 103.075) (end 119.15 104.7) (width 0.25) (layer F.Cu) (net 7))
 (segment (start 122.149 100.076) (end 119.15 103.075) (width 0.25) (layer F.Cu) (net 7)))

